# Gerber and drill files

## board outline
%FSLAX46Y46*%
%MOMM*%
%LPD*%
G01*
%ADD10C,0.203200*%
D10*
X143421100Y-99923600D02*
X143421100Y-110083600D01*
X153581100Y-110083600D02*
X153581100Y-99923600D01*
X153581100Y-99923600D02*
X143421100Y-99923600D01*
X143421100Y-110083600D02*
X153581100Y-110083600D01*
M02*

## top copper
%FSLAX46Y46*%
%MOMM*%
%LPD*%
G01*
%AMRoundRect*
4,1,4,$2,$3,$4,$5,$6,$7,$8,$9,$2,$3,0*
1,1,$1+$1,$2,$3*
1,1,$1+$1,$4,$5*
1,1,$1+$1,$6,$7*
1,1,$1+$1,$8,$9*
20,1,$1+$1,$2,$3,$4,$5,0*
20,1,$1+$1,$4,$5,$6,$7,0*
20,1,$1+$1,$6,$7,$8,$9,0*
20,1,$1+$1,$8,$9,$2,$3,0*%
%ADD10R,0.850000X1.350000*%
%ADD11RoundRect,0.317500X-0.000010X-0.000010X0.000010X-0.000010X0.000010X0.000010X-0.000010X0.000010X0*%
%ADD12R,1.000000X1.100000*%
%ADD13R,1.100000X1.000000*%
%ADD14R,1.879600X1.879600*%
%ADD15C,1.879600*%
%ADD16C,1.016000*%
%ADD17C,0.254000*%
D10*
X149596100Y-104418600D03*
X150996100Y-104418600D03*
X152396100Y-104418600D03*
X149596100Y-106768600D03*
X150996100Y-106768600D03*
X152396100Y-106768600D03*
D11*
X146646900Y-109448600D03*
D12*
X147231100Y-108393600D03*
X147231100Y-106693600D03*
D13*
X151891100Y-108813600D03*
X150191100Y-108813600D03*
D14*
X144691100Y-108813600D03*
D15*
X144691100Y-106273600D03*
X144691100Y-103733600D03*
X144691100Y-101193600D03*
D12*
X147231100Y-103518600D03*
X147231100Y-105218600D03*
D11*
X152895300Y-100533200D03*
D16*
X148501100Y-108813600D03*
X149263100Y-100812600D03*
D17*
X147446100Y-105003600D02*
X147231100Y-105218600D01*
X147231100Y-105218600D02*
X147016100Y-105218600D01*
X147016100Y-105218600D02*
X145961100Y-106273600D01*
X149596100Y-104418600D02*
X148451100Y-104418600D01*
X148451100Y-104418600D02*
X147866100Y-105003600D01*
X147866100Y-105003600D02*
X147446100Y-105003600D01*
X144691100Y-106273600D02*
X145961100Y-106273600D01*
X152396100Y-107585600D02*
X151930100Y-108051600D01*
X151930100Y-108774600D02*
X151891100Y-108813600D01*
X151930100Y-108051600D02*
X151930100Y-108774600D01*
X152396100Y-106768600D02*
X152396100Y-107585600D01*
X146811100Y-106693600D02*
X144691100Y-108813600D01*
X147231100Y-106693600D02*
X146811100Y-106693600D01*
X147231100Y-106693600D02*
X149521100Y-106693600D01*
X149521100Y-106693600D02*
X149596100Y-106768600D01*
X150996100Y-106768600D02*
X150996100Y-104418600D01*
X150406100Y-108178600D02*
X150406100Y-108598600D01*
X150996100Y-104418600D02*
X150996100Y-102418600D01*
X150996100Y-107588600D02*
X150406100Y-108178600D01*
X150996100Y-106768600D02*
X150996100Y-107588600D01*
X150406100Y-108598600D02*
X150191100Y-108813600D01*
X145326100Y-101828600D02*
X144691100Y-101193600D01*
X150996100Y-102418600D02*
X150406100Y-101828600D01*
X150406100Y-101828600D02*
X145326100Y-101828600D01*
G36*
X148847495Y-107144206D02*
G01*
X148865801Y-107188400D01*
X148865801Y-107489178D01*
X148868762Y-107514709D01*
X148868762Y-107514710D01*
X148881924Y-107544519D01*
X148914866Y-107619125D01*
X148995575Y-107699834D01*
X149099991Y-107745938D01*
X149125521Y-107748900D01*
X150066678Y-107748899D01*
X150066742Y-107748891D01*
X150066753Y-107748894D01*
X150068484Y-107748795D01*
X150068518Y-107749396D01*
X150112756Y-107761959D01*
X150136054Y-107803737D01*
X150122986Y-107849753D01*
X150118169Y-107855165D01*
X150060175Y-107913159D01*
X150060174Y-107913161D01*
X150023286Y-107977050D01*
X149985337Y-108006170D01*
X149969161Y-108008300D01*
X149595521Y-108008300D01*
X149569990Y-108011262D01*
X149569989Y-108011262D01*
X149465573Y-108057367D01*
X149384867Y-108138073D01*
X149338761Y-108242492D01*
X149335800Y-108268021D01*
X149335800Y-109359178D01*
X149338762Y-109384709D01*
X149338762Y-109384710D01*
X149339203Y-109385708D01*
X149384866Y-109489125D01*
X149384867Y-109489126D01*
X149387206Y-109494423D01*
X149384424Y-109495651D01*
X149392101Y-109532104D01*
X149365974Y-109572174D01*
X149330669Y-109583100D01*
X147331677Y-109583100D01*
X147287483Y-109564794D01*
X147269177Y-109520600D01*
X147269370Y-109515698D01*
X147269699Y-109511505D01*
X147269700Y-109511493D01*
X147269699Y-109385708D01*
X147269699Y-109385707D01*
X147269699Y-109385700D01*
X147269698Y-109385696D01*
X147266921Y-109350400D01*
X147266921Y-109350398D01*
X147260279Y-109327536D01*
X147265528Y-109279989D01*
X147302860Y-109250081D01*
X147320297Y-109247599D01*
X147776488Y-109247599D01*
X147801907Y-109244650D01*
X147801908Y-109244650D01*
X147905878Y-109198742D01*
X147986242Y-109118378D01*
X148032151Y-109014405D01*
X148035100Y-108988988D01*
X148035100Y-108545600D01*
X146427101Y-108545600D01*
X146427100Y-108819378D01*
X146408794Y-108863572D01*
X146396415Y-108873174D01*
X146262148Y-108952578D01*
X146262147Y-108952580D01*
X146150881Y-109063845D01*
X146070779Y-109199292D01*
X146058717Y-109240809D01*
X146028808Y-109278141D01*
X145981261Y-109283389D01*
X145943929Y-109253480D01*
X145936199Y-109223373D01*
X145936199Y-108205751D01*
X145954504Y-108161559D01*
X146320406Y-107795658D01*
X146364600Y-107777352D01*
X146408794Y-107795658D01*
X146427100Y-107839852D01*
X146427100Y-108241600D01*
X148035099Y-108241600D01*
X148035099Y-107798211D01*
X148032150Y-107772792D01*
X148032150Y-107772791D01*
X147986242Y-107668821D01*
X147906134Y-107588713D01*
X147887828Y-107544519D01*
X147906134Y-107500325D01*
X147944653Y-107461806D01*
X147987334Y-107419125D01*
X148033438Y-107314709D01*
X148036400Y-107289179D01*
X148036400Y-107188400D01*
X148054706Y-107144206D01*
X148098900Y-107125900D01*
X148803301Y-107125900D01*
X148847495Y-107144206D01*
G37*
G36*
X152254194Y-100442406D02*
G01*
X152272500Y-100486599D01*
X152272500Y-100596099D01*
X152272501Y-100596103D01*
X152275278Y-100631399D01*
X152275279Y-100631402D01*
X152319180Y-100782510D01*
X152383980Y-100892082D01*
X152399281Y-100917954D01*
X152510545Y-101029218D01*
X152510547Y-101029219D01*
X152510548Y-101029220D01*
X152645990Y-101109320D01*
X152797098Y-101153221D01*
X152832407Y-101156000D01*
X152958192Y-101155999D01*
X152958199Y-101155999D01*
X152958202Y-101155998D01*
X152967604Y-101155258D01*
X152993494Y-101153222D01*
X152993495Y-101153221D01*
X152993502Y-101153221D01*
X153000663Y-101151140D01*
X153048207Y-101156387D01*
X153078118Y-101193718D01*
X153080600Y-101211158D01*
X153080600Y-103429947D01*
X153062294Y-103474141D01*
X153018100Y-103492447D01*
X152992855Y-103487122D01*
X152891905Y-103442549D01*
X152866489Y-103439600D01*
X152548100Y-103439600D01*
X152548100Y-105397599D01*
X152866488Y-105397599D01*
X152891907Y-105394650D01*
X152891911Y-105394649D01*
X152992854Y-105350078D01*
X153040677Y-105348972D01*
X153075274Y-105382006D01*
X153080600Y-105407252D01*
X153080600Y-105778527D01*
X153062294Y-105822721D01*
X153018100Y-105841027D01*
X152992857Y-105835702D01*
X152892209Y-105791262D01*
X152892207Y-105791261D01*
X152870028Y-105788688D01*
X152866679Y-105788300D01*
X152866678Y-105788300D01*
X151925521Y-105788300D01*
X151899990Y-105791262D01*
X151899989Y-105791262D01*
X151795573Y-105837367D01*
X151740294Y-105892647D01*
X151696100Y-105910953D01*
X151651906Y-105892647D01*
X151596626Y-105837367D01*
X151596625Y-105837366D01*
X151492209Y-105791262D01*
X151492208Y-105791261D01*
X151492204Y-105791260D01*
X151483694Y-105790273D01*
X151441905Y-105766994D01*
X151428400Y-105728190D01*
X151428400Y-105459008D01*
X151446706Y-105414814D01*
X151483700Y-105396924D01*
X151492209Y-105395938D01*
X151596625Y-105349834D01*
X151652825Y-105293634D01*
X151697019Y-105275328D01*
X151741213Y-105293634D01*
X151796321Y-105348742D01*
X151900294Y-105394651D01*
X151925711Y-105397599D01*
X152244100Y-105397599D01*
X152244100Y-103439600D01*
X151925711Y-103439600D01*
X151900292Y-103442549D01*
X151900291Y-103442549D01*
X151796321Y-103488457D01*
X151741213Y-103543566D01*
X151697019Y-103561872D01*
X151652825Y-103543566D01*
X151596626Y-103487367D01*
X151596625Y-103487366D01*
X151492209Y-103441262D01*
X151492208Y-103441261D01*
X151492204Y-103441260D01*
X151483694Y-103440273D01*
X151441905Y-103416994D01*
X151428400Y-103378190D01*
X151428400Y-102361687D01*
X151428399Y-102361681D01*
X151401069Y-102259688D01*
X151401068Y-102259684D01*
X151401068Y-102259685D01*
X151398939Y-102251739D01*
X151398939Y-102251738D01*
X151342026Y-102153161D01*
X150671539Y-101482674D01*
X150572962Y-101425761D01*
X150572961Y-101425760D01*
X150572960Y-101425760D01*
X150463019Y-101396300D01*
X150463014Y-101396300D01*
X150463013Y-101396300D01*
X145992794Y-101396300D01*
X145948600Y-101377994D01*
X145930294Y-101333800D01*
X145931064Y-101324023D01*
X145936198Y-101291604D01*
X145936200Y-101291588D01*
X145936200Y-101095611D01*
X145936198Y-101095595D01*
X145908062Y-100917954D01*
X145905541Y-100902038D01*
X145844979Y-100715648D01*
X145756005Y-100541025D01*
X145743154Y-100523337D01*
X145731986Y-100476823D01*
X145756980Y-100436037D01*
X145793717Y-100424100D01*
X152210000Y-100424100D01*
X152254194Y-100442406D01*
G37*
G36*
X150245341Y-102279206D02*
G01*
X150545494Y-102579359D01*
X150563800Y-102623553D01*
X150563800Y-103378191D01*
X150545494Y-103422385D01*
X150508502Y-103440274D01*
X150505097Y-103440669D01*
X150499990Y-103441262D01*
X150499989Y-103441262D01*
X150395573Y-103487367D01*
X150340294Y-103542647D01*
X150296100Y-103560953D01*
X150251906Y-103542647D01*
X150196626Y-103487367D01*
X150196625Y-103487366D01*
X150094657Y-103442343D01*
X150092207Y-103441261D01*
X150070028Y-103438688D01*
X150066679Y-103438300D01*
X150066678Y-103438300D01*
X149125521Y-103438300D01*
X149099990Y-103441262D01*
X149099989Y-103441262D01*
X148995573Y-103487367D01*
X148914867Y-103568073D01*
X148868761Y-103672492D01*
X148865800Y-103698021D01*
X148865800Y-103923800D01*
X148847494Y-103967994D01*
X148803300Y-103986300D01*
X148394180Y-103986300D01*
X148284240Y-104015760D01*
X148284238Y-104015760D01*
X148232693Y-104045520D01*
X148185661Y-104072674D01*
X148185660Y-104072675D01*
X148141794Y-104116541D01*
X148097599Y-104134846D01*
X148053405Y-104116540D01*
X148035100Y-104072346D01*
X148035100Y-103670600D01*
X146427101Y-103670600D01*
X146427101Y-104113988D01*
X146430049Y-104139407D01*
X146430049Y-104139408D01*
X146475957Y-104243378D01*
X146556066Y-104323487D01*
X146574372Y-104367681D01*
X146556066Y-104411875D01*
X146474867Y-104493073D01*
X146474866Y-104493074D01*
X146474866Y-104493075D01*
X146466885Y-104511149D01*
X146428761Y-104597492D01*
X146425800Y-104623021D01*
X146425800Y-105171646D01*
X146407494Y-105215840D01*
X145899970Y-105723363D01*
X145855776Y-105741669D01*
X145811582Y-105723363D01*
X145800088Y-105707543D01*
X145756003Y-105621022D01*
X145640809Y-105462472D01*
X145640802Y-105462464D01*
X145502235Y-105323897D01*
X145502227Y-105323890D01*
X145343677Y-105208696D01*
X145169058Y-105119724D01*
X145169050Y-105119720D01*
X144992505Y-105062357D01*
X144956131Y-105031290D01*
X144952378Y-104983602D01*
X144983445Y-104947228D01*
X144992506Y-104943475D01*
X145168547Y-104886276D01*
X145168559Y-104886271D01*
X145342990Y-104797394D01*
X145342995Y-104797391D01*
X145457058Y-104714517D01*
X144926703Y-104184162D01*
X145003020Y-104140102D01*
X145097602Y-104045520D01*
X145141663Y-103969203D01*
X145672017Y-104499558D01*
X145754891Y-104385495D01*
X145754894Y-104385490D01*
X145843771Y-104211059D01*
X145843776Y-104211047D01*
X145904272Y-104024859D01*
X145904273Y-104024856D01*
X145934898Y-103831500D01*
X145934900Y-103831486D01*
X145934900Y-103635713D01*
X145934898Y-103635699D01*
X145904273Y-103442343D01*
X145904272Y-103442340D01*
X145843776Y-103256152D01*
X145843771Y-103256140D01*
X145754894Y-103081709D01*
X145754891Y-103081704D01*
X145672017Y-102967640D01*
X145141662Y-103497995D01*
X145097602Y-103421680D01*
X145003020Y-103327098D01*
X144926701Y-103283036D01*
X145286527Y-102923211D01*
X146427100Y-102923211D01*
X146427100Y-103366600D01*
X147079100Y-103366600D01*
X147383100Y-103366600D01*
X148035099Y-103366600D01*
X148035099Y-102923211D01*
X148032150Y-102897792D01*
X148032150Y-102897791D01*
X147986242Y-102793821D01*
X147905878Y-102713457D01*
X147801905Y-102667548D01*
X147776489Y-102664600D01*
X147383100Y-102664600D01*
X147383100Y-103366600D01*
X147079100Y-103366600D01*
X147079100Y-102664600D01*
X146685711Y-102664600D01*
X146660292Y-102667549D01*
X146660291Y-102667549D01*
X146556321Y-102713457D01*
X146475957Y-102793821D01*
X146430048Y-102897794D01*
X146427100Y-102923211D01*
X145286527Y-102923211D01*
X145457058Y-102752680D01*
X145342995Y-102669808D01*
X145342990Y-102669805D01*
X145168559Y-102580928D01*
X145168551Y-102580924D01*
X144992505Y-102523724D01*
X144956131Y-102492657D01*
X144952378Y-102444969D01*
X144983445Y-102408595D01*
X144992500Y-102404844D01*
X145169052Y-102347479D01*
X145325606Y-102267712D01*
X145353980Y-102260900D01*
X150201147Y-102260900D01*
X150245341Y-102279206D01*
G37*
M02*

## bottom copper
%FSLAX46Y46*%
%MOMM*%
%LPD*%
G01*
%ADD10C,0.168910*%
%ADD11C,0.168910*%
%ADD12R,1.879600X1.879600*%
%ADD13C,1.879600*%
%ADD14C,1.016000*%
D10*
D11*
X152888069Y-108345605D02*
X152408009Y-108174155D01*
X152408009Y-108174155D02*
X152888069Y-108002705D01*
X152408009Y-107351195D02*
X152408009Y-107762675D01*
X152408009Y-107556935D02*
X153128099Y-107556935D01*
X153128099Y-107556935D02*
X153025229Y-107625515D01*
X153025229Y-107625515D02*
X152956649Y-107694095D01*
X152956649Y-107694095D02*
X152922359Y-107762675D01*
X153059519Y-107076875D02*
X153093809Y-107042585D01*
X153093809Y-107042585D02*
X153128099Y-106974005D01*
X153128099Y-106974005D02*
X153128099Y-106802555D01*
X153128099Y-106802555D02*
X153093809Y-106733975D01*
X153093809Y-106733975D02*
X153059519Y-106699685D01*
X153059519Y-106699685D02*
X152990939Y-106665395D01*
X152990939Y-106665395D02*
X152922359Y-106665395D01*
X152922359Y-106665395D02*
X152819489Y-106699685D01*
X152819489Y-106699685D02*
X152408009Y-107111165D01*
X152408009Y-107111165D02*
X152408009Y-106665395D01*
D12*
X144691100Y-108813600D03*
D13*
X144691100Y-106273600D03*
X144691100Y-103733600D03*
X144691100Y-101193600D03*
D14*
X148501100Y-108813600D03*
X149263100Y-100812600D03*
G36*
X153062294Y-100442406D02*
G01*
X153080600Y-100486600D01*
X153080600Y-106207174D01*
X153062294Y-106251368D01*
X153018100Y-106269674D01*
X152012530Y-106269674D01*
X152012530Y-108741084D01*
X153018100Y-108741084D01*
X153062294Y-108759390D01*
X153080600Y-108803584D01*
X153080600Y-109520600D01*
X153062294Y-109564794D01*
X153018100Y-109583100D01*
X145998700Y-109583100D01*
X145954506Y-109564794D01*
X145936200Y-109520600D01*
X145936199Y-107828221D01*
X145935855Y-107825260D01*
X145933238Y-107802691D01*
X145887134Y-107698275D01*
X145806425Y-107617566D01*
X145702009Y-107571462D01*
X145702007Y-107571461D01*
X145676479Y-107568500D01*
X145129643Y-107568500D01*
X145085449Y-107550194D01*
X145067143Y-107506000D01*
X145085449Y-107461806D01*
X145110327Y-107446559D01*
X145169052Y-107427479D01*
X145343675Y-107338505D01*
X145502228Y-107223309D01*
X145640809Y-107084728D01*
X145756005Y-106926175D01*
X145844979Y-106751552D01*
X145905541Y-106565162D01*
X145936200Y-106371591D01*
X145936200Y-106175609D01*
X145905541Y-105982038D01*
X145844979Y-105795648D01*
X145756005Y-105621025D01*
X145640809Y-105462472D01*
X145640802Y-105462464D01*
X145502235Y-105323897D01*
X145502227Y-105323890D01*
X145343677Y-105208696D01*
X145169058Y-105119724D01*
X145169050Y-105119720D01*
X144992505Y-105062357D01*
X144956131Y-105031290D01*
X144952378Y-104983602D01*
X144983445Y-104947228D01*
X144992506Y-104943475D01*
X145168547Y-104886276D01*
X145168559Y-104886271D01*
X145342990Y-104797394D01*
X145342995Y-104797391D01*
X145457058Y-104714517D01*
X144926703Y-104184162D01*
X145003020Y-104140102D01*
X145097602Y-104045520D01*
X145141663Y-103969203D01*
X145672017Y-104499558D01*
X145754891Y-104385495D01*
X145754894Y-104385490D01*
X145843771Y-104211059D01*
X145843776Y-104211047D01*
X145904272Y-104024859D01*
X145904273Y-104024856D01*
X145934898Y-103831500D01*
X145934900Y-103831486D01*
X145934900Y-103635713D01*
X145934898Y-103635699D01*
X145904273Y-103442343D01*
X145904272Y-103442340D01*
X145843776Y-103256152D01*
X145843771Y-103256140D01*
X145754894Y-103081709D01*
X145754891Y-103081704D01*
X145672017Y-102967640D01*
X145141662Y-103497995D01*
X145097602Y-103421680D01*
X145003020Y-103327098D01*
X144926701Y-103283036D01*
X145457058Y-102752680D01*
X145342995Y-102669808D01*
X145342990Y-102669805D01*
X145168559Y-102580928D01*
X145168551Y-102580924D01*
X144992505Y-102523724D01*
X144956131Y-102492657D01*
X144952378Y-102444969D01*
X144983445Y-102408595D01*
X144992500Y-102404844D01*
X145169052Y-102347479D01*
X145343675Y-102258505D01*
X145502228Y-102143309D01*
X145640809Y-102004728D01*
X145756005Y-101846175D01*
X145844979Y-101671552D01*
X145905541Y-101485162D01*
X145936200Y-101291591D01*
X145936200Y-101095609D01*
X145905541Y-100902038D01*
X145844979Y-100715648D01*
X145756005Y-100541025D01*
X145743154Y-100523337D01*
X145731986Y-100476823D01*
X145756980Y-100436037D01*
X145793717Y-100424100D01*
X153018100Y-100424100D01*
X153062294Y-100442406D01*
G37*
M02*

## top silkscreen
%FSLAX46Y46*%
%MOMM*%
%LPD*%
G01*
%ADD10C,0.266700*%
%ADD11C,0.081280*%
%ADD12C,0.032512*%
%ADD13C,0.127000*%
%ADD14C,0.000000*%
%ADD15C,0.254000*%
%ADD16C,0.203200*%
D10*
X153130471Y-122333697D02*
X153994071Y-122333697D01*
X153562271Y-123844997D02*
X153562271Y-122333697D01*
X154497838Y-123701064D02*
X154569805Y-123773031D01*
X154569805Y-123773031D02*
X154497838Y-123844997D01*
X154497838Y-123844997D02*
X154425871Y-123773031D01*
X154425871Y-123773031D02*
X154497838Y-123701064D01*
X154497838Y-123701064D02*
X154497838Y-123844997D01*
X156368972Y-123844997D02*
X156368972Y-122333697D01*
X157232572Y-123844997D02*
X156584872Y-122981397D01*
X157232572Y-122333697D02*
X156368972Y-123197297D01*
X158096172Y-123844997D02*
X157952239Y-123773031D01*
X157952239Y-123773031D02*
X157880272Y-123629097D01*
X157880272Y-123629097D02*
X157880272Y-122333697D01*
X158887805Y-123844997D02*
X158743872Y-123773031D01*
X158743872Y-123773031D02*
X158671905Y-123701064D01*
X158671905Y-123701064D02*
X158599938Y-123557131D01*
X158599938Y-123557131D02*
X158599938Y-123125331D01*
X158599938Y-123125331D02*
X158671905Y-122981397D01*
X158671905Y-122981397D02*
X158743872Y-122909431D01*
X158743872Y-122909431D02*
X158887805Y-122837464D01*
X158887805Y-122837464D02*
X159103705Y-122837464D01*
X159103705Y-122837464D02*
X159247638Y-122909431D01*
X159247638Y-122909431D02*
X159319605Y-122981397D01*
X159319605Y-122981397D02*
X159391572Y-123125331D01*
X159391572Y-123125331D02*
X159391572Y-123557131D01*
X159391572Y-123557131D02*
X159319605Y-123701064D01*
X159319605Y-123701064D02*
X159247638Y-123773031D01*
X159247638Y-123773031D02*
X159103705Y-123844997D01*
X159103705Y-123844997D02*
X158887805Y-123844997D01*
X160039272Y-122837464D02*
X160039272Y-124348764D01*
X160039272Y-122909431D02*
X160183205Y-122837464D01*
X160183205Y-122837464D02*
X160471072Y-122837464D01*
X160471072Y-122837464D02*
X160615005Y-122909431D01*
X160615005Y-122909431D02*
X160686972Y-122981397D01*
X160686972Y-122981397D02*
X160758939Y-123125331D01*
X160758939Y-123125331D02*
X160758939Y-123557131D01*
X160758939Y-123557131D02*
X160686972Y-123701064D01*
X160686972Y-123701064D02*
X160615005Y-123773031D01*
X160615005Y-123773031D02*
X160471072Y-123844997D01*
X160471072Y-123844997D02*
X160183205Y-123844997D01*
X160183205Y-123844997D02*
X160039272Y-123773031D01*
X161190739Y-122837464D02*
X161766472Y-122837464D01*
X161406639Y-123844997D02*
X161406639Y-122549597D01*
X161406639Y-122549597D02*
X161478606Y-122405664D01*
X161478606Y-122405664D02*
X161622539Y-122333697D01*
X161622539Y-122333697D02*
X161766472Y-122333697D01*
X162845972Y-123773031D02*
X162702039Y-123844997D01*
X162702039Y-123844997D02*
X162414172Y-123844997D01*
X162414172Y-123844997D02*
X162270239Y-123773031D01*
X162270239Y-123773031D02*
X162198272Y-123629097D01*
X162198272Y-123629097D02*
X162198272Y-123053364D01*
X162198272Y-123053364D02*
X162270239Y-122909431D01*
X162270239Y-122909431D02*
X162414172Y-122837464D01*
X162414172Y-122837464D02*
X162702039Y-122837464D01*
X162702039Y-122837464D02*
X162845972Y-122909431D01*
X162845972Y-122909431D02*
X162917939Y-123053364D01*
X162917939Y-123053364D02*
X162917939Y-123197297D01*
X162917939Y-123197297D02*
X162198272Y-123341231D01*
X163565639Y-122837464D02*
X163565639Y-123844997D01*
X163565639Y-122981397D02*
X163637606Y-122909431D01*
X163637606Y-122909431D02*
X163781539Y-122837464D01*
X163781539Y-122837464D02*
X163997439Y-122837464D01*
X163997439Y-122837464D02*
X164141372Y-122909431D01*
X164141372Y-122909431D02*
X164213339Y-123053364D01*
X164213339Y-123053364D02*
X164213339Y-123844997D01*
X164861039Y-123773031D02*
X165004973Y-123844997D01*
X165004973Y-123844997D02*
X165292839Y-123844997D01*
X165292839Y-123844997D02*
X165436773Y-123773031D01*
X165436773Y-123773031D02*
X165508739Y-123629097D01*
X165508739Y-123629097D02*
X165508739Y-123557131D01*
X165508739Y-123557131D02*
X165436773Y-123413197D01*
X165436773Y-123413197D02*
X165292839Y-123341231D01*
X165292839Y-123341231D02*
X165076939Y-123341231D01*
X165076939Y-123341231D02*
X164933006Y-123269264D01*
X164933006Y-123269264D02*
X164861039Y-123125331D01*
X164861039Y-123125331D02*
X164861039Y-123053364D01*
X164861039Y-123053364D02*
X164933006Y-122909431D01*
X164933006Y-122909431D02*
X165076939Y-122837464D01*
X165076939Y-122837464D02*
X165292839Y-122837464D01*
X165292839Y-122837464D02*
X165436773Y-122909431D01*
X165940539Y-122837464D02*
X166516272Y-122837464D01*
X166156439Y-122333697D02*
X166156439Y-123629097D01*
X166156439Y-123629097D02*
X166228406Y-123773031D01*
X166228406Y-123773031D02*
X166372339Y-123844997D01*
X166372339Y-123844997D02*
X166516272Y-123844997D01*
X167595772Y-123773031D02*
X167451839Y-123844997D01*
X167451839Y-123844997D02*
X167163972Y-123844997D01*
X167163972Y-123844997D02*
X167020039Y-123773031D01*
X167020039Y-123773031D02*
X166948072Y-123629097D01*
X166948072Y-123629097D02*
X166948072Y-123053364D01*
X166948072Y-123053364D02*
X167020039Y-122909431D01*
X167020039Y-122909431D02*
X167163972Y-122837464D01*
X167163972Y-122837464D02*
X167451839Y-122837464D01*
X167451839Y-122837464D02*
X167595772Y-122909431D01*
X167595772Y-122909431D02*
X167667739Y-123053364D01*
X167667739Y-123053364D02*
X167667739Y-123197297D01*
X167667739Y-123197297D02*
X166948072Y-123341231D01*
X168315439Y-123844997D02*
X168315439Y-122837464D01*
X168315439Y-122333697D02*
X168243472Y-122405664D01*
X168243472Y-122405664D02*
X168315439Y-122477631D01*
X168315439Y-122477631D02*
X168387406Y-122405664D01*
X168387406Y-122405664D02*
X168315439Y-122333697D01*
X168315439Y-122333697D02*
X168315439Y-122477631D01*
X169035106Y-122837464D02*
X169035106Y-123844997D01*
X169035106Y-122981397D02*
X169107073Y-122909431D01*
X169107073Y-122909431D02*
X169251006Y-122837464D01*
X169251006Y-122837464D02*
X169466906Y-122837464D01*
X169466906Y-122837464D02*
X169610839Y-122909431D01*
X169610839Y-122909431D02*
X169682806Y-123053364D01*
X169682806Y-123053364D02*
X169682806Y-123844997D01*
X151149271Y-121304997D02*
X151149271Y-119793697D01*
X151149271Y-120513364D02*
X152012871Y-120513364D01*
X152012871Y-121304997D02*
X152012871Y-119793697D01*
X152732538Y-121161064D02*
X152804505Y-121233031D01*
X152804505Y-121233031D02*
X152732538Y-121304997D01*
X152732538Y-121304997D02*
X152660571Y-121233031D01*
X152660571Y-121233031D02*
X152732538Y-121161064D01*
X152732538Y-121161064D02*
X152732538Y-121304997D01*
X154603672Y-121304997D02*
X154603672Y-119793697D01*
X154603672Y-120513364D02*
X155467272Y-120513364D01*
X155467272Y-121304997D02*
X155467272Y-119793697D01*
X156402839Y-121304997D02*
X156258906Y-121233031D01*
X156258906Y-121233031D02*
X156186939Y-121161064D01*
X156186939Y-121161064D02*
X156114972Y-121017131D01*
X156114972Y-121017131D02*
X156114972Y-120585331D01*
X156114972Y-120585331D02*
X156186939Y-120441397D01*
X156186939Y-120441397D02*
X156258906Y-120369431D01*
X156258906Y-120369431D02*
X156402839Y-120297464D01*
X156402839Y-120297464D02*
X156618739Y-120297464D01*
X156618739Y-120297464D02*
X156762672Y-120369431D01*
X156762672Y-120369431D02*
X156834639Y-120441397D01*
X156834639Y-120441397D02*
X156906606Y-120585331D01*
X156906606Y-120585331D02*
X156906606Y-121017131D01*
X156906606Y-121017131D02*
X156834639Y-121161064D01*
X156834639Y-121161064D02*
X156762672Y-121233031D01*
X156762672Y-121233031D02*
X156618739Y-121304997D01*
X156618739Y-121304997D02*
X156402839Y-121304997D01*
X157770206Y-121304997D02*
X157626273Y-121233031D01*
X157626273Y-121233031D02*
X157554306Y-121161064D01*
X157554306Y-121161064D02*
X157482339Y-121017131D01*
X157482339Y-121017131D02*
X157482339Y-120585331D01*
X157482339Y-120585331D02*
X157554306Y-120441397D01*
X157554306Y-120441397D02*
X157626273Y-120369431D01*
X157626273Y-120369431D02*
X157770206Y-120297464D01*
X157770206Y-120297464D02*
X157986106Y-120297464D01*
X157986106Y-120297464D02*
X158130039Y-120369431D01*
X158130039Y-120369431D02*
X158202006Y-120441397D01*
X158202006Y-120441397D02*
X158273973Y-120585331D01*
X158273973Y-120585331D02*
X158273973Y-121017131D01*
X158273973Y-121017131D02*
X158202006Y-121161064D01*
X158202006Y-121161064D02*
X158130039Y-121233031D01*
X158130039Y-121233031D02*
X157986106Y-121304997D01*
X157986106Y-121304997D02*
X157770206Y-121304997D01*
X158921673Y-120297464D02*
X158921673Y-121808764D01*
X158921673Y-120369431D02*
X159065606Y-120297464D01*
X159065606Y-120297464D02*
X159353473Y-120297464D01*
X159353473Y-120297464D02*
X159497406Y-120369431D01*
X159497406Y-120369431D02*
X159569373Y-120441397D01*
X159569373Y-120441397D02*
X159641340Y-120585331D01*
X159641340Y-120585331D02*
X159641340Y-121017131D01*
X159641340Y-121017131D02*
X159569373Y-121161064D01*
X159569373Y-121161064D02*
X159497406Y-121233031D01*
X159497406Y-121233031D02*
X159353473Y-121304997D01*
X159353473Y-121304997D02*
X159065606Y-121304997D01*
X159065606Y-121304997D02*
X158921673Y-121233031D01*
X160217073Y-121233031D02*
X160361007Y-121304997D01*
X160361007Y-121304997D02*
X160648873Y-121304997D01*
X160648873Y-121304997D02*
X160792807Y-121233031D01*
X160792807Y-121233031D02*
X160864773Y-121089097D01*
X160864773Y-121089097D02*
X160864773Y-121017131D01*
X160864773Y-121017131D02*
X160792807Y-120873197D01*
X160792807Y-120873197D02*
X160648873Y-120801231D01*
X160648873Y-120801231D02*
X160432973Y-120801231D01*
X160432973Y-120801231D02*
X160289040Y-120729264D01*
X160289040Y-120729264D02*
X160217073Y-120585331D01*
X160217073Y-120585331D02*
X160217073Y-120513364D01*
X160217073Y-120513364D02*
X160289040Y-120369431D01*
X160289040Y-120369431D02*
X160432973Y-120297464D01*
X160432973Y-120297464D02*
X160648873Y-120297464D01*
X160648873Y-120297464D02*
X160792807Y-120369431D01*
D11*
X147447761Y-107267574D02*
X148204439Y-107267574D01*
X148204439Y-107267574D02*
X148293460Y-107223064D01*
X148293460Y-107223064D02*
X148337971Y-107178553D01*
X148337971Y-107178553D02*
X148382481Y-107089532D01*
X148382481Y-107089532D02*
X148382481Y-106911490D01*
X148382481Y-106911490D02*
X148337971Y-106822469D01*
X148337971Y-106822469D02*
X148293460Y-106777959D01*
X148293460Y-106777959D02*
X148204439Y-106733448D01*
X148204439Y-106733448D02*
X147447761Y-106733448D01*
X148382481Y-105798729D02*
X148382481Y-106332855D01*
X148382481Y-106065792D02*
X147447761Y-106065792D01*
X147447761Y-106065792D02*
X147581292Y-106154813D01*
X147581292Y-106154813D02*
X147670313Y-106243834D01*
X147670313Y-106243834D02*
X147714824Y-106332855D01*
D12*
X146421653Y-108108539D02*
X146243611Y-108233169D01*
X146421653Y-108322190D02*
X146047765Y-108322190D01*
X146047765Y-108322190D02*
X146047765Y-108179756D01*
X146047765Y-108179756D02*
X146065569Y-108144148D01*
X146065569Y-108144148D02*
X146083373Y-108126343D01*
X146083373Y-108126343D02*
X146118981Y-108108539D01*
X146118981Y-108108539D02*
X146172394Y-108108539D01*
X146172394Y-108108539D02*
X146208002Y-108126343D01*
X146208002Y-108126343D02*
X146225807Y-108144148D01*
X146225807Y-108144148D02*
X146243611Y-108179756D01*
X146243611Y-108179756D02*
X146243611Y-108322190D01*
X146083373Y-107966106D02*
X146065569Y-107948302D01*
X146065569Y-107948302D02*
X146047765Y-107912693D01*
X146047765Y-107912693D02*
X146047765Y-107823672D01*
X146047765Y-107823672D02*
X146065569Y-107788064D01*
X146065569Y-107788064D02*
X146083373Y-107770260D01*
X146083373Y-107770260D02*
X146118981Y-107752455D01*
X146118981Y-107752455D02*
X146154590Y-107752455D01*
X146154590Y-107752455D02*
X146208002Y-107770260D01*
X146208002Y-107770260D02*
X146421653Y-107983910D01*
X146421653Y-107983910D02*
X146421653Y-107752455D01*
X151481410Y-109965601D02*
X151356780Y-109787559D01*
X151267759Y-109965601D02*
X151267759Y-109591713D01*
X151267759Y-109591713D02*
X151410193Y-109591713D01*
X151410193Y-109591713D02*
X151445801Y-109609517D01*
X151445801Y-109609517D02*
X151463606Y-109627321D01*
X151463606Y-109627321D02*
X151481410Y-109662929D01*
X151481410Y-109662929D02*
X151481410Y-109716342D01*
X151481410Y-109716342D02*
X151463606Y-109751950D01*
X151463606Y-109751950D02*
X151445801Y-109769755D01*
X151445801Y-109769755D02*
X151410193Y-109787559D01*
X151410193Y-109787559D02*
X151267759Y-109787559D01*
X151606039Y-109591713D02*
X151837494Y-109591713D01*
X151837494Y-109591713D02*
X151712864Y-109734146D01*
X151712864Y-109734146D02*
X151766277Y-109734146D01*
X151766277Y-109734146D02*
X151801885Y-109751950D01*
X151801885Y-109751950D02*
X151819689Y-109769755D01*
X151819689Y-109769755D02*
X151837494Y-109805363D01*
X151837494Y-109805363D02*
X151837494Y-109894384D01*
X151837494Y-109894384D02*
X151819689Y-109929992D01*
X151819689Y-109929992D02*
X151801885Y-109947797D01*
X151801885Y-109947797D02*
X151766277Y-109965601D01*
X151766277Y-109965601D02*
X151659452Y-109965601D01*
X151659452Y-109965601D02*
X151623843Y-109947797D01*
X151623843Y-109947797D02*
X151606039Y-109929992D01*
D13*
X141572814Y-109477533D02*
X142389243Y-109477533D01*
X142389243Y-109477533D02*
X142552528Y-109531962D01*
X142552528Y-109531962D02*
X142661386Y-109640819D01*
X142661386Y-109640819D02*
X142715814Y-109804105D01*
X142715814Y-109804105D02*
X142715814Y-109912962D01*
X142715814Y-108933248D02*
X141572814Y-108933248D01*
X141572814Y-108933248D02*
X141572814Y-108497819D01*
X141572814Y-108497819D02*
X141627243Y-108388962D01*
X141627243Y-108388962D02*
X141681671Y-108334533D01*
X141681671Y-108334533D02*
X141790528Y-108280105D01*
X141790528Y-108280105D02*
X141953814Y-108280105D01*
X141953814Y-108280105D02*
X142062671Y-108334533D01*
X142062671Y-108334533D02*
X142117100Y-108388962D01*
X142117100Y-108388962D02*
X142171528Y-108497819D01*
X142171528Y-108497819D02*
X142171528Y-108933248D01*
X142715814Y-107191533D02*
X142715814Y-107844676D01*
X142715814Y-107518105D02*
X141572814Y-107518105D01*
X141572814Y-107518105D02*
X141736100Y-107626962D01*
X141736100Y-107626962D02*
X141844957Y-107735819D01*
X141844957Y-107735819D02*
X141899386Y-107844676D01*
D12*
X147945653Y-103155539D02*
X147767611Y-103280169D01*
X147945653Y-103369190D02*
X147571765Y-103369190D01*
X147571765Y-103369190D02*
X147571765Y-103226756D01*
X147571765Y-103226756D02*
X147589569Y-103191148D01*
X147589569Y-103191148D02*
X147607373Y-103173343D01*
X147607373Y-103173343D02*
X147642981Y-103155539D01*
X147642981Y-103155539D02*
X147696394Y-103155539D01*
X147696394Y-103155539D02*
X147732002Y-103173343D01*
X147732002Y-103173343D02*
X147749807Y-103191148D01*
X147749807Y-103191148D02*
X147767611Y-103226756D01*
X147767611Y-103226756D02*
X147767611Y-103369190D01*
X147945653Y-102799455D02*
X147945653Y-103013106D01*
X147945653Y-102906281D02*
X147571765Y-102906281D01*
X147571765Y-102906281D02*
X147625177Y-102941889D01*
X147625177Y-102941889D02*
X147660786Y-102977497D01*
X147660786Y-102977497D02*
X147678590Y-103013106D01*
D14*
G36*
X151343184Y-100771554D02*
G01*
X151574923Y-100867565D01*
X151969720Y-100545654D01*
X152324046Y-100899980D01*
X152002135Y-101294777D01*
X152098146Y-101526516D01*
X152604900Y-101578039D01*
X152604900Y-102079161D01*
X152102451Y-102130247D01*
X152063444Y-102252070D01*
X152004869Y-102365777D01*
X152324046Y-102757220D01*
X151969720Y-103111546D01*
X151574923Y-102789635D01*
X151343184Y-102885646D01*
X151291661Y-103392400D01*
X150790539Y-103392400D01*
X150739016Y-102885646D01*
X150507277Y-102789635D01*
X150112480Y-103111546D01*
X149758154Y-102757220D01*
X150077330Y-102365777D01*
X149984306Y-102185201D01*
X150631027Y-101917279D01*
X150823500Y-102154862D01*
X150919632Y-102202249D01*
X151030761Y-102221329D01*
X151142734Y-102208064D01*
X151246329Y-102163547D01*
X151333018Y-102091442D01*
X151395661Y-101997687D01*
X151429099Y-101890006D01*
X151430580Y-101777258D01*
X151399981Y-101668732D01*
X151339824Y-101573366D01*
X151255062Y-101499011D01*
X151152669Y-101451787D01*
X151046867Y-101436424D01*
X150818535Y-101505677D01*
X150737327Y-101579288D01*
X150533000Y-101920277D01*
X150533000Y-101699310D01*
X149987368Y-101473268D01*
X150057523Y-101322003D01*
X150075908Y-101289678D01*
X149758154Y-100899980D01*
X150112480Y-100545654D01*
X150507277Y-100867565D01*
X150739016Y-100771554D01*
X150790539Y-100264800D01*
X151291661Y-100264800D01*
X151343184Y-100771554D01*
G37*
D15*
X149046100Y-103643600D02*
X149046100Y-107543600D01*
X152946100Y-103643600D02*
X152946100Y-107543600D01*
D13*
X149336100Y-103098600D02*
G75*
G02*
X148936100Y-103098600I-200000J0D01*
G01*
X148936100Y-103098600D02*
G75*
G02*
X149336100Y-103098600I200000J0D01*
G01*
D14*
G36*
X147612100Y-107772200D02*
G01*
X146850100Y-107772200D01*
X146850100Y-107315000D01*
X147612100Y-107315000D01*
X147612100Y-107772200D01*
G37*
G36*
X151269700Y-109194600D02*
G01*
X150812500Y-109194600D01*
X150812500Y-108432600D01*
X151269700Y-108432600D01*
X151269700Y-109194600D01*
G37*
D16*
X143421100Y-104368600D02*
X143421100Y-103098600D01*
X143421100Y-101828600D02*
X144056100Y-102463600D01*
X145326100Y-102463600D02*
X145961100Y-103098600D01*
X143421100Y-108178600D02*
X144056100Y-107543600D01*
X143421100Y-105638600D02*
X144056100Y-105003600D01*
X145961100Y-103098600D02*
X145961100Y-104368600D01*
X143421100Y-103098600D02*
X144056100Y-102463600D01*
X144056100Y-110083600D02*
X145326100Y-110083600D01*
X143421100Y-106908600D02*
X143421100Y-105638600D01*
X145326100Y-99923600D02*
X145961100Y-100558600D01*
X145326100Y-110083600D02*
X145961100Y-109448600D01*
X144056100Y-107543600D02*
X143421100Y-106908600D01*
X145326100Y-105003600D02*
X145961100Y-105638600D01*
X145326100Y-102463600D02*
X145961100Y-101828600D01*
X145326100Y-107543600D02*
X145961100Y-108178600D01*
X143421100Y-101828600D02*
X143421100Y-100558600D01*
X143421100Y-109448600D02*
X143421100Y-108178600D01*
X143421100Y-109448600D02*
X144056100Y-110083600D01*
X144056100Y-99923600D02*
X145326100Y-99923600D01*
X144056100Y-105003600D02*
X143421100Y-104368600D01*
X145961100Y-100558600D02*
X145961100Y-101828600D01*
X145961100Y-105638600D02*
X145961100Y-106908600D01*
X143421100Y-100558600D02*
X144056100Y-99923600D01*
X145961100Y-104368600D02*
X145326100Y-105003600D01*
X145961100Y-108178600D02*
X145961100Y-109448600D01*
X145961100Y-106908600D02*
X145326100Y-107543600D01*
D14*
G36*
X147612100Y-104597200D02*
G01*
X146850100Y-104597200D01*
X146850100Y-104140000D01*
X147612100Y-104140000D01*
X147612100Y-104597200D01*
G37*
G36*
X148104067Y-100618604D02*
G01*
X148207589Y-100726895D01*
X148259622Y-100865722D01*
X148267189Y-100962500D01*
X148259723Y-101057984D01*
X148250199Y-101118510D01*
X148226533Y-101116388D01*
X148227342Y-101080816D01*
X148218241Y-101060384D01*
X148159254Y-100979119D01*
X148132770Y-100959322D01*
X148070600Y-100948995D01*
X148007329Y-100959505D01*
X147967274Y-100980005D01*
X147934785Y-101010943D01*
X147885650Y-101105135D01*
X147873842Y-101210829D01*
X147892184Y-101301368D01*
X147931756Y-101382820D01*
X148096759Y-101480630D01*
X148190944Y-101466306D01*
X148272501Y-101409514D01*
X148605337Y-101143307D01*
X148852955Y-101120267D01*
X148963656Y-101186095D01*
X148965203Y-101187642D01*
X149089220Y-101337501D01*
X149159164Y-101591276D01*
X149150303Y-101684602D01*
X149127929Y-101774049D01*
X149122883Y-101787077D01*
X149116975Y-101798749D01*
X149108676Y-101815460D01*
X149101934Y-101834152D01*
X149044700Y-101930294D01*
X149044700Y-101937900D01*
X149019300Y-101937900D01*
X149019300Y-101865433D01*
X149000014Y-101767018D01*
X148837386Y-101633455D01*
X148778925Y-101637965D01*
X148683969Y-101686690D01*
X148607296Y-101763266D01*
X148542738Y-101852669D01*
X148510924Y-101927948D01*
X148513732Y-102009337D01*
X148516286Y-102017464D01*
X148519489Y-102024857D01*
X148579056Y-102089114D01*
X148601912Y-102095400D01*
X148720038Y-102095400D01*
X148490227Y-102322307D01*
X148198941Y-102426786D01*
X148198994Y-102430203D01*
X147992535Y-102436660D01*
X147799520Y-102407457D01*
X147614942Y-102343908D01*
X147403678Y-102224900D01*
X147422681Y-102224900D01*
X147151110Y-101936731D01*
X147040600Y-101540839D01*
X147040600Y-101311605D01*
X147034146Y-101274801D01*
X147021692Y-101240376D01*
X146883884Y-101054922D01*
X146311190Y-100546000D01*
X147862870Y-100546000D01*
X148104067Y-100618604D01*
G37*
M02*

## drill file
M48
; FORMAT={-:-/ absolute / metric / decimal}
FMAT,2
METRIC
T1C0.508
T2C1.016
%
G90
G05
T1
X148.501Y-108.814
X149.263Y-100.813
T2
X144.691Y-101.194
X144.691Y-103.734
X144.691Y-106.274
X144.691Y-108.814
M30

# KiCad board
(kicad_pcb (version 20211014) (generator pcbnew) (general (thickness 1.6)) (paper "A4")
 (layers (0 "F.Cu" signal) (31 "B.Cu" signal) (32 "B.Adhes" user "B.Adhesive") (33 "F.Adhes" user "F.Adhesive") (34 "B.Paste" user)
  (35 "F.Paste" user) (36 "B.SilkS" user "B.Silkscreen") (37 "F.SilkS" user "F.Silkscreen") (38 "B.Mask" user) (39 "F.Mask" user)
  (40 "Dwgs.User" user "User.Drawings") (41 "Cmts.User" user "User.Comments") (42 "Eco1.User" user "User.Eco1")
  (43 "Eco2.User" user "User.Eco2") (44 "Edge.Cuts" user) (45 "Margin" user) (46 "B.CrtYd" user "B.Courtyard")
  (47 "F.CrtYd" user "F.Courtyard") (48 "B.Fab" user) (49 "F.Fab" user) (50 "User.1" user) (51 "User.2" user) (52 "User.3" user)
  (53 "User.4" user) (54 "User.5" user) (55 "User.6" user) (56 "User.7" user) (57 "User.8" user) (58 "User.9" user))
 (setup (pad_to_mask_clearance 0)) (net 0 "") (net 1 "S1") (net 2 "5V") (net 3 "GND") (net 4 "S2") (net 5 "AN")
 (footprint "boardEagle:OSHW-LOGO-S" (layer "F.Cu") (at 151.0411 101.8286 -90)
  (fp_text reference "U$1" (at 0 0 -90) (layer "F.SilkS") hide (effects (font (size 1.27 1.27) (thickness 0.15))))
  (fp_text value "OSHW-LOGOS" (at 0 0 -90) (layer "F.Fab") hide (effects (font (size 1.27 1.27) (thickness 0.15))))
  (fp_poly
   (pts (xy 0.301647 -1.061351) (xy 0.42347 -1.022344) (xy 0.537177 -0.963769) (xy 0.92862 -1.282946) (xy 1.282946 -0.92862)
    (xy 0.961035 -0.533823) (xy 1.057046 -0.302084) (xy 1.5638 -0.250561) (xy 1.5638 0.250561) (xy 1.057046 0.302084) (xy 0.961035 0.533823)
    (xy 1.282946 0.92862) (xy 0.92862 1.282946) (xy 0.537177 0.96377) (xy 0.356601 1.056794) (xy 0.088679 0.410073) (xy 0.326262 0.2176)
    (xy 0.373649 0.121468) (xy 0.392729 0.010339) (xy 0.379464 -0.101634) (xy 0.334947 -0.205229) (xy 0.262842 -0.291918)
    (xy 0.169087 -0.354561) (xy 0.061406 -0.387999) (xy -0.051342 -0.38948) (xy -0.159868 -0.358881) (xy -0.255234 -0.298724)
    (xy -0.329589 -0.213962) (xy -0.376813 -0.111569) (xy -0.392176 -0.005767) (xy -0.322923 0.222565) (xy -0.249312 0.303773)
    (xy 0.091677 0.5081) (xy -0.12929 0.5081) (xy -0.355332 1.053732) (xy -0.506597 0.983577) (xy -0.538922 0.965192) (xy -0.92862 1.282946)
    (xy -1.282946 0.92862) (xy -0.961035 0.533823) (xy -1.057046 0.302084) (xy -1.5638 0.250561) (xy -1.5638 -0.250561)
    (xy -1.057046 -0.302084) (xy -0.961035 -0.533823) (xy -1.282946 -0.92862) (xy -0.92862 -1.282946) (xy -0.533823 -0.961035)
    (xy -0.302084 -1.057046) (xy -0.250561 -1.5638) (xy 0.250561 -1.5638))
   (layer "F.SilkS") (width 0) (fill solid)))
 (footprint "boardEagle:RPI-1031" (layer "F.Cu") (at 151.0411 105.6386 90)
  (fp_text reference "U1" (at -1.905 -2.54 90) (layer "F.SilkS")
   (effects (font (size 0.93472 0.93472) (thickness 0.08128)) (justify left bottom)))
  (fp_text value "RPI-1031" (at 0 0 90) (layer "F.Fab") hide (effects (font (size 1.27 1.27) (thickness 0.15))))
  (fp_line (start 1.995 -1.995) (end -1.905 -1.995) (layer "F.SilkS") (width 0.254))
  (fp_line (start 1.995 1.905) (end -1.905 1.905) (layer "F.SilkS") (width 0.254))
  (fp_circle (center 2.54 -1.905) (end 2.74 -1.905) (layer "F.SilkS") (width 0.127) (fill none))
  (pad "1" smd rect (at 1.22 -1.445 180) (size 0.85 1.35) (layers "F.Cu" "F.Paste" "F.Mask") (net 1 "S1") (solder_mask_margin 0.1016))
  (pad "2" smd rect (at 1.22 -0.045 180) (size 0.85 1.35) (layers "F.Cu" "F.Paste" "F.Mask") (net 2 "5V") (solder_mask_margin 0.1016))
  (pad "3" smd rect (at 1.22 1.355 180) (size 0.85 1.35) (layers "F.Cu" "F.Paste" "F.Mask") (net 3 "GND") (solder_mask_margin 0.1016))
  (pad "4" smd rect (at -1.13 -1.445 180) (size 0.85 1.35) (layers "F.Cu" "F.Paste" "F.Mask") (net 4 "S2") (solder_mask_margin 0.1016))
  (pad "5" smd rect (at -1.13 -0.045 180) (size 0.85 1.35) (layers "F.Cu" "F.Paste" "F.Mask") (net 2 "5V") (solder_mask_margin 0.1016))
  (pad "6" smd rect (at -1.13 1.355 180) (size 0.85 1.35) (layers "F.Cu" "F.Paste" "F.Mask") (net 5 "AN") (solder_mask_margin 0.1016)))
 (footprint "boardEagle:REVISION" (layer "F.Cu") (at 129.4511 124.0536)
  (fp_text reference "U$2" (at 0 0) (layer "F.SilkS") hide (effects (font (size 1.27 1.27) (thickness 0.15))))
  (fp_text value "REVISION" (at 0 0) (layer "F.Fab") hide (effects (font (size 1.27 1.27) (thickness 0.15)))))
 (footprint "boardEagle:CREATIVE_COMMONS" (layer "F.Cu") (at 118.548979 121.5136)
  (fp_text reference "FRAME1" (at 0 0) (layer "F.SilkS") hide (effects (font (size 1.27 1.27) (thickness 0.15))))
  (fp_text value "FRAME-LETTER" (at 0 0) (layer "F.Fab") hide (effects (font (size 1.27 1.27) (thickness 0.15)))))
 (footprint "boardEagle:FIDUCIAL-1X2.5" (layer "F.Cu") (at 146.6469 109.4486)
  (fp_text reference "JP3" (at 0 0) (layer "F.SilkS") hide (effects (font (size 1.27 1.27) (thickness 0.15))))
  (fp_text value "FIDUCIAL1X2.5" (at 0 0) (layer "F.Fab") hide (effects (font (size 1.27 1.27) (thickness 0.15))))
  (pad "1" smd roundrect (at 0 0) (size 0.635 0.635) (layers "F.Cu" "F.Mask") (roundrect_rratio 0.5) (solder_mask_margin 0.1016)))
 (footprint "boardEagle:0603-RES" (layer "F.Cu") (at 147.2311 107.5436 90)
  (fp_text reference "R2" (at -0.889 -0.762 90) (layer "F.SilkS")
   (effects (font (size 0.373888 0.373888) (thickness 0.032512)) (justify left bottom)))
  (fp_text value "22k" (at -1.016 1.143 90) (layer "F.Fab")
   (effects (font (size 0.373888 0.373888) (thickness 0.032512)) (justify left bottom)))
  (fp_poly (pts (xy -0.2286 0.381) (xy 0.2286 0.381) (xy 0.2286 -0.381) (xy -0.2286 -0.381)) (layer "F.SilkS") (width 0) (fill solid))
  (pad "1" smd rect (at -0.85 0 90) (size 1.1 1) (layers "F.Cu" "F.Paste" "F.Mask") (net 3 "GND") (solder_mask_margin 0.1016))
  (pad "2" smd rect (at 0.85 0 90) (size 1.1 1) (layers "F.Cu" "F.Paste" "F.Mask") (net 4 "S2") (solder_mask_margin 0.1016)))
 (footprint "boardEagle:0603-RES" (layer "F.Cu") (at 151.0411 108.8136 180)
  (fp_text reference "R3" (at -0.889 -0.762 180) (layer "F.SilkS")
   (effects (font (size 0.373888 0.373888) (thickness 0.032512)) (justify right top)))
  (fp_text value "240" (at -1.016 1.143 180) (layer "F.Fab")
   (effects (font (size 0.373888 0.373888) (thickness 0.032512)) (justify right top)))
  (fp_poly (pts (xy -0.2286 0.381) (xy 0.2286 0.381) (xy 0.2286 -0.381) (xy -0.2286 -0.381)) (layer "F.SilkS") (width 0) (fill solid))
  (pad "1" smd rect (at -0.85 0 180) (size 1.1 1) (layers "F.Cu" "F.Paste" "F.Mask") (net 5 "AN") (solder_mask_margin 0.1016))
  (pad "2" smd rect (at 0.85 0 180) (size 1.1 1) (layers "F.Cu" "F.Paste" "F.Mask") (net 2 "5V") (solder_mask_margin 0.1016)))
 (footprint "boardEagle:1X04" (layer "F.Cu") (at 144.6911 108.8136 90)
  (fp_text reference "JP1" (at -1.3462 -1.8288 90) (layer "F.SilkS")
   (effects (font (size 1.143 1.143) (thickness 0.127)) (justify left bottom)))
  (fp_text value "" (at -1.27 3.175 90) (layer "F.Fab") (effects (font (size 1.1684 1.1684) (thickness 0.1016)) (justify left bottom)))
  (fp_line (start 4.445 -1.27) (end 5.715 -1.27) (layer "F.SilkS") (width 0.2032))
  (fp_line (start 6.985 -1.27) (end 6.35 -0.635) (layer "F.SilkS") (width 0.2032))
  (fp_line (start 6.35 0.635) (end 5.715 1.27) (layer "F.SilkS") (width 0.2032))
  (fp_line (start 0.635 -1.27) (end 1.27 -0.635) (layer "F.SilkS") (width 0.2032))
  (fp_line (start 3.175 -1.27) (end 3.81 -0.635) (layer "F.SilkS") (width 0.2032))
  (fp_line (start 5.715 1.27) (end 4.445 1.27) (layer "F.SilkS") (width 0.2032))
  (fp_line (start 5.715 -1.27) (end 6.35 -0.635) (layer "F.SilkS") (width 0.2032))
  (fp_line (start -1.27 -0.635) (end -1.27 0.635) (layer "F.SilkS") (width 0.2032))
  (fp_line (start 1.905 -1.27) (end 3.175 -1.27) (layer "F.SilkS") (width 0.2032))
  (fp_line (start 8.89 0.635) (end 8.255 1.27) (layer "F.SilkS") (width 0.2032))
  (fp_line (start -1.27 0.635) (end -0.635 1.27) (layer "F.SilkS") (width 0.2032))
  (fp_line (start 1.27 -0.635) (end 1.905 -1.27) (layer "F.SilkS") (width 0.2032))
  (fp_line (start 3.81 0.635) (end 3.175 1.27) (layer "F.SilkS") (width 0.2032))
  (fp_line (start 6.35 0.635) (end 6.985 1.27) (layer "F.SilkS") (width 0.2032))
  (fp_line (start 1.27 0.635) (end 0.635 1.27) (layer "F.SilkS") (width 0.2032))
  (fp_line (start 6.985 -1.27) (end 8.255 -1.27) (layer "F.SilkS") (width 0.2032))
  (fp_line (start -0.635 -1.27) (end 0.635 -1.27) (layer "F.SilkS") (width 0.2032))
  (fp_line (start -0.635 -1.27) (end -1.27 -0.635) (layer "F.SilkS") (width 0.2032))
  (fp_line (start 8.89 -0.635) (end 8.89 0.635) (layer "F.SilkS") (width 0.2032))
  (fp_line (start 3.81 -0.635) (end 4.445 -1.27) (layer "F.SilkS") (width 0.2032))
  (fp_line (start 8.255 1.27) (end 6.985 1.27) (layer "F.SilkS") (width 0.2032))
  (fp_line (start 3.175 1.27) (end 1.905 1.27) (layer "F.SilkS") (width 0.2032))
  (fp_line (start 8.255 -1.27) (end 8.89 -0.635) (layer "F.SilkS") (width 0.2032))
  (fp_line (start 4.445 1.27) (end 3.81 0.635) (layer "F.SilkS") (width 0.2032))
  (fp_line (start 0.635 1.27) (end -0.635 1.27) (layer "F.SilkS") (width 0.2032))
  (fp_line (start 1.905 1.27) (end 1.27 0.635) (layer "F.SilkS") (width 0.2032))
  (pad "1" thru_hole rect (at 0 0 180) (size 1.8796 1.8796) (drill 1.016) (layers *.Cu *.Mask) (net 4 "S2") (solder_mask_margin 0.1016))
  (pad "2" thru_hole circle (at 2.54 0 180) (size 1.8796 1.8796) (drill 1.016) (layers *.Cu *.Mask) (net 1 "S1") (solder_mask_margin 0.1016))
  (pad "3" thru_hole circle (at 5.08 0 180) (size 1.8796 1.8796) (drill 1.016) (layers *.Cu *.Mask) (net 3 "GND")
   (solder_mask_margin 0.1016))
  (pad "4" thru_hole circle (at 7.62 0 180) (size 1.8796 1.8796) (drill 1.016) (layers *.Cu *.Mask) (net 2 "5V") (solder_mask_margin 0.1016)))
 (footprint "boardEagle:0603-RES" (layer "F.Cu") (at 147.2311 104.3686 -90)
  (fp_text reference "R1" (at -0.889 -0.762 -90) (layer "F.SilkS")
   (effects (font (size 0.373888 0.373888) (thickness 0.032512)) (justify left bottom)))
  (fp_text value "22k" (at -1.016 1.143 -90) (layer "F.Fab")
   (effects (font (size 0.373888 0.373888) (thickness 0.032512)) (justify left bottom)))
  (fp_poly (pts (xy -0.2286 0.381) (xy 0.2286 0.381) (xy 0.2286 -0.381) (xy -0.2286 -0.381)) (layer "F.SilkS") (width 0) (fill solid))
  (pad "1" smd rect (at -0.85 0 270) (size 1.1 1) (layers "F.Cu" "F.Paste" "F.Mask") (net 3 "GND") (solder_mask_margin 0.1016))
  (pad "2" smd rect (at 0.85 0 270) (size 1.1 1) (layers "F.Cu" "F.Paste" "F.Mask") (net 1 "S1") (solder_mask_margin 0.1016)))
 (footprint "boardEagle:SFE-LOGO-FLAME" (layer "F.Cu") (at 146.3421 100.5586 -90)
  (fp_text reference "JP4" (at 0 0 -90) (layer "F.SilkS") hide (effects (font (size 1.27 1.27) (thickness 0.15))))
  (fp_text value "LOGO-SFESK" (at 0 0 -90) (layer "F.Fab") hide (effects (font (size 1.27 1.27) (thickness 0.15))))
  (fp_poly
   (pts (xy 1.126002 -2.808203) (xy 1.215449 -2.785829) (xy 1.228477 -2.780783) (xy 1.240149 -2.774875) (xy 1.25686 -2.766576)
    (xy 1.275552 -2.759834) (xy 1.371694 -2.7026) (xy 1.3793 -2.7026) (xy 1.3793 -2.6772) (xy 1.306833 -2.6772) (xy 1.208418 -2.657914)
    (xy 1.074855 -2.495286) (xy 1.079365 -2.436825) (xy 1.12809 -2.341869) (xy 1.204666 -2.265196) (xy 1.294069 -2.200638)
    (xy 1.369348 -2.168824) (xy 1.450737 -2.171632) (xy 1.458864 -2.174186) (xy 1.466257 -2.177389) (xy 1.530514 -2.236956)
    (xy 1.5368 -2.259812) (xy 1.5368 -2.377938) (xy 1.763707 -2.148127) (xy 1.868186 -1.856841) (xy 1.871603 -1.856894)
    (xy 1.87806 -1.650435) (xy 1.848857 -1.45742) (xy 1.785308 -1.272842) (xy 1.6663 -1.061578) (xy 1.6663 -1.080581) (xy 1.378131 -0.80901)
    (xy 0.982239 -0.6985) (xy 0.753005 -0.6985) (xy 0.716201 -0.692046) (xy 0.681776 -0.679592) (xy 0.496322 -0.541784) (xy -0.0126 0.03091)
    (xy -0.0126 -1.52077) (xy 0.060004 -1.761967) (xy 0.168295 -1.865489) (xy 0.307122 -1.917522) (xy 0.4039 -1.925089)
    (xy 0.499384 -1.917623) (xy 0.55991 -1.908099) (xy 0.557788 -1.884433) (xy 0.522216 -1.885242) (xy 0.501784 -1.876141)
    (xy 0.420519 -1.817154) (xy 0.400722 -1.79067) (xy 0.390395 -1.7285) (xy 0.400905 -1.665229) (xy 0.421405 -1.625174)
    (xy 0.452343 -1.592685) (xy 0.546535 -1.54355) (xy 0.652229 -1.531742) (xy 0.742768 -1.550084) (xy 0.82422 -1.589656)
    (xy 0.92203 -1.754659) (xy 0.907706 -1.848844) (xy 0.850914 -1.930401) (xy 0.584707 -2.263237) (xy 0.561667 -2.510855)
    (xy 0.627495 -2.621556) (xy 0.629042 -2.623103) (xy 0.778901 -2.74712) (xy 1.032676 -2.817064))
   (layer "F.SilkS") (width 0) (fill solid)))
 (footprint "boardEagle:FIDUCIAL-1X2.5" (layer "F.Cu") (at 152.8953 100.5332)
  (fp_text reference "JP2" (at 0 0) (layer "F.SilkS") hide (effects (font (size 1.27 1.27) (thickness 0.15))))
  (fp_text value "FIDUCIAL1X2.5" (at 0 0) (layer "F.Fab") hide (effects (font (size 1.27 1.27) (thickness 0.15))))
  (pad "1" smd roundrect (at 0 0) (size 0.635 0.635) (layers "F.Cu" "F.Mask") (roundrect_rratio 0.5) (solder_mask_margin 0.1016)))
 (gr_line (start 143.4211 99.9236) (end 143.4211 110.0836) (layer "Edge.Cuts") (width 0.2032))
 (gr_line (start 153.5811 110.0836) (end 153.5811 99.9236) (layer "Edge.Cuts") (width 0.2032))
 (gr_line (start 153.5811 99.9236) (end 143.4211 99.9236) (layer "Edge.Cuts") (width 0.2032))
 (gr_line (start 143.4211 110.0836) (end 153.5811 110.0836) (layer "Edge.Cuts") (width 0.2032))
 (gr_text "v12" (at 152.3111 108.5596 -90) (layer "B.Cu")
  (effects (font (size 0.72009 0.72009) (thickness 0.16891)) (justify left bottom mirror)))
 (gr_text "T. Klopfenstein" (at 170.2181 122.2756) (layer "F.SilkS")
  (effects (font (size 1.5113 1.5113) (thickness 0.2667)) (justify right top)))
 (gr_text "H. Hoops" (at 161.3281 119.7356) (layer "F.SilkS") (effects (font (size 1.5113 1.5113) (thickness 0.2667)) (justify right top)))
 (via (at 148.5011 108.8136) (size 1.016) (drill 0.508) (layers "F.Cu" "B.Cu") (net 3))
 (via (at 149.2631 100.8126) (size 1.016) (drill 0.508) (layers "F.Cu" "B.Cu") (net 3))
 (segment (start 147.4461 105.0036) (end 147.2311 105.2186) (width 0.254) (layer "F.Cu") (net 1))
 (segment (start 147.2311 105.2186) (end 147.0161 105.2186) (width 0.254) (layer "F.Cu") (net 1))
 (segment (start 147.0161 105.2186) (end 145.9611 106.2736) (width 0.254) (layer "F.Cu") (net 1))
 (segment (start 149.5961 104.4186) (end 148.4511 104.4186) (width 0.254) (layer "F.Cu") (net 1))
 (segment (start 148.4511 104.4186) (end 147.8661 105.0036) (width 0.254) (layer "F.Cu") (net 1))
 (segment (start 147.8661 105.0036) (end 147.4461 105.0036) (width 0.254) (layer "F.Cu") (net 1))
 (segment (start 144.6911 106.2736) (end 145.9611 106.2736) (width 0.254) (layer "F.Cu") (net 1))
 (segment (start 152.3961 107.5856) (end 151.9301 108.0516) (width 0.254) (layer "F.Cu") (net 5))
 (segment (start 151.9301 108.7746) (end 151.8911 108.8136) (width 0.254) (layer "F.Cu") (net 5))
 (segment (start 151.9301 108.0516) (end 151.9301 108.7746) (width 0.254) (layer "F.Cu") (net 5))
 (segment (start 152.3961 106.7686) (end 152.3961 107.5856) (width 0.254) (layer "F.Cu") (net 5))
 (segment (start 146.8111 106.6936) (end 144.6911 108.8136) (width 0.254) (layer "F.Cu") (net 4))
 (segment (start 147.2311 106.6936) (end 146.8111 106.6936) (width 0.254) (layer "F.Cu") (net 4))
 (segment (start 147.2311 106.6936) (end 149.5211 106.6936) (width 0.254) (layer "F.Cu") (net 4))
 (segment (start 149.5211 106.6936) (end 149.5961 106.7686) (width 0.254) (layer "F.Cu") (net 4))
 (segment (start 150.9961 106.7686) (end 150.9961 104.4186) (width 0.254) (layer "F.Cu") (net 2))
 (segment (start 150.4061 108.1786) (end 150.4061 108.5986) (width 0.254) (layer "F.Cu") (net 2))
 (segment (start 150.9961 104.4186) (end 150.9961 102.4186) (width 0.254) (layer "F.Cu") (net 2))
 (segment (start 150.9961 107.5886) (end 150.4061 108.1786) (width 0.254) (layer "F.Cu") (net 2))
 (segment (start 150.9961 106.7686) (end 150.9961 107.5886) (width 0.254) (layer "F.Cu") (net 2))
 (segment (start 150.4061 108.5986) (end 150.1911 108.8136) (width 0.254) (layer "F.Cu") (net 2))
 (segment (start 145.3261 101.8286) (end 144.6911 101.1936) (width 0.254) (layer "F.Cu") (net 2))
 (segment (start 150.9961 102.4186) (end 150.4061 101.8286) (width 0.254) (layer "F.Cu") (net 2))
 (segment (start 150.4061 101.8286) (end 145.3261 101.8286) (width 0.254) (layer "F.Cu") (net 2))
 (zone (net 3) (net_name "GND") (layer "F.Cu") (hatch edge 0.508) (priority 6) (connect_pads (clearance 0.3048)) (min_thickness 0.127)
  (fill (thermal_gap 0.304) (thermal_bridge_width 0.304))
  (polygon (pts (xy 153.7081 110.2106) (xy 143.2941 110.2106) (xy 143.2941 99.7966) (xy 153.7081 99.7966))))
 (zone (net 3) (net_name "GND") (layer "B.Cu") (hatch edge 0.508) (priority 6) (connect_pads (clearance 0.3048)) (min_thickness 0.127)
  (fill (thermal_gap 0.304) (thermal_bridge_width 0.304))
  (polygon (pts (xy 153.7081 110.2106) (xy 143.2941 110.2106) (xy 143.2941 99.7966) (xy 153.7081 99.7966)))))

